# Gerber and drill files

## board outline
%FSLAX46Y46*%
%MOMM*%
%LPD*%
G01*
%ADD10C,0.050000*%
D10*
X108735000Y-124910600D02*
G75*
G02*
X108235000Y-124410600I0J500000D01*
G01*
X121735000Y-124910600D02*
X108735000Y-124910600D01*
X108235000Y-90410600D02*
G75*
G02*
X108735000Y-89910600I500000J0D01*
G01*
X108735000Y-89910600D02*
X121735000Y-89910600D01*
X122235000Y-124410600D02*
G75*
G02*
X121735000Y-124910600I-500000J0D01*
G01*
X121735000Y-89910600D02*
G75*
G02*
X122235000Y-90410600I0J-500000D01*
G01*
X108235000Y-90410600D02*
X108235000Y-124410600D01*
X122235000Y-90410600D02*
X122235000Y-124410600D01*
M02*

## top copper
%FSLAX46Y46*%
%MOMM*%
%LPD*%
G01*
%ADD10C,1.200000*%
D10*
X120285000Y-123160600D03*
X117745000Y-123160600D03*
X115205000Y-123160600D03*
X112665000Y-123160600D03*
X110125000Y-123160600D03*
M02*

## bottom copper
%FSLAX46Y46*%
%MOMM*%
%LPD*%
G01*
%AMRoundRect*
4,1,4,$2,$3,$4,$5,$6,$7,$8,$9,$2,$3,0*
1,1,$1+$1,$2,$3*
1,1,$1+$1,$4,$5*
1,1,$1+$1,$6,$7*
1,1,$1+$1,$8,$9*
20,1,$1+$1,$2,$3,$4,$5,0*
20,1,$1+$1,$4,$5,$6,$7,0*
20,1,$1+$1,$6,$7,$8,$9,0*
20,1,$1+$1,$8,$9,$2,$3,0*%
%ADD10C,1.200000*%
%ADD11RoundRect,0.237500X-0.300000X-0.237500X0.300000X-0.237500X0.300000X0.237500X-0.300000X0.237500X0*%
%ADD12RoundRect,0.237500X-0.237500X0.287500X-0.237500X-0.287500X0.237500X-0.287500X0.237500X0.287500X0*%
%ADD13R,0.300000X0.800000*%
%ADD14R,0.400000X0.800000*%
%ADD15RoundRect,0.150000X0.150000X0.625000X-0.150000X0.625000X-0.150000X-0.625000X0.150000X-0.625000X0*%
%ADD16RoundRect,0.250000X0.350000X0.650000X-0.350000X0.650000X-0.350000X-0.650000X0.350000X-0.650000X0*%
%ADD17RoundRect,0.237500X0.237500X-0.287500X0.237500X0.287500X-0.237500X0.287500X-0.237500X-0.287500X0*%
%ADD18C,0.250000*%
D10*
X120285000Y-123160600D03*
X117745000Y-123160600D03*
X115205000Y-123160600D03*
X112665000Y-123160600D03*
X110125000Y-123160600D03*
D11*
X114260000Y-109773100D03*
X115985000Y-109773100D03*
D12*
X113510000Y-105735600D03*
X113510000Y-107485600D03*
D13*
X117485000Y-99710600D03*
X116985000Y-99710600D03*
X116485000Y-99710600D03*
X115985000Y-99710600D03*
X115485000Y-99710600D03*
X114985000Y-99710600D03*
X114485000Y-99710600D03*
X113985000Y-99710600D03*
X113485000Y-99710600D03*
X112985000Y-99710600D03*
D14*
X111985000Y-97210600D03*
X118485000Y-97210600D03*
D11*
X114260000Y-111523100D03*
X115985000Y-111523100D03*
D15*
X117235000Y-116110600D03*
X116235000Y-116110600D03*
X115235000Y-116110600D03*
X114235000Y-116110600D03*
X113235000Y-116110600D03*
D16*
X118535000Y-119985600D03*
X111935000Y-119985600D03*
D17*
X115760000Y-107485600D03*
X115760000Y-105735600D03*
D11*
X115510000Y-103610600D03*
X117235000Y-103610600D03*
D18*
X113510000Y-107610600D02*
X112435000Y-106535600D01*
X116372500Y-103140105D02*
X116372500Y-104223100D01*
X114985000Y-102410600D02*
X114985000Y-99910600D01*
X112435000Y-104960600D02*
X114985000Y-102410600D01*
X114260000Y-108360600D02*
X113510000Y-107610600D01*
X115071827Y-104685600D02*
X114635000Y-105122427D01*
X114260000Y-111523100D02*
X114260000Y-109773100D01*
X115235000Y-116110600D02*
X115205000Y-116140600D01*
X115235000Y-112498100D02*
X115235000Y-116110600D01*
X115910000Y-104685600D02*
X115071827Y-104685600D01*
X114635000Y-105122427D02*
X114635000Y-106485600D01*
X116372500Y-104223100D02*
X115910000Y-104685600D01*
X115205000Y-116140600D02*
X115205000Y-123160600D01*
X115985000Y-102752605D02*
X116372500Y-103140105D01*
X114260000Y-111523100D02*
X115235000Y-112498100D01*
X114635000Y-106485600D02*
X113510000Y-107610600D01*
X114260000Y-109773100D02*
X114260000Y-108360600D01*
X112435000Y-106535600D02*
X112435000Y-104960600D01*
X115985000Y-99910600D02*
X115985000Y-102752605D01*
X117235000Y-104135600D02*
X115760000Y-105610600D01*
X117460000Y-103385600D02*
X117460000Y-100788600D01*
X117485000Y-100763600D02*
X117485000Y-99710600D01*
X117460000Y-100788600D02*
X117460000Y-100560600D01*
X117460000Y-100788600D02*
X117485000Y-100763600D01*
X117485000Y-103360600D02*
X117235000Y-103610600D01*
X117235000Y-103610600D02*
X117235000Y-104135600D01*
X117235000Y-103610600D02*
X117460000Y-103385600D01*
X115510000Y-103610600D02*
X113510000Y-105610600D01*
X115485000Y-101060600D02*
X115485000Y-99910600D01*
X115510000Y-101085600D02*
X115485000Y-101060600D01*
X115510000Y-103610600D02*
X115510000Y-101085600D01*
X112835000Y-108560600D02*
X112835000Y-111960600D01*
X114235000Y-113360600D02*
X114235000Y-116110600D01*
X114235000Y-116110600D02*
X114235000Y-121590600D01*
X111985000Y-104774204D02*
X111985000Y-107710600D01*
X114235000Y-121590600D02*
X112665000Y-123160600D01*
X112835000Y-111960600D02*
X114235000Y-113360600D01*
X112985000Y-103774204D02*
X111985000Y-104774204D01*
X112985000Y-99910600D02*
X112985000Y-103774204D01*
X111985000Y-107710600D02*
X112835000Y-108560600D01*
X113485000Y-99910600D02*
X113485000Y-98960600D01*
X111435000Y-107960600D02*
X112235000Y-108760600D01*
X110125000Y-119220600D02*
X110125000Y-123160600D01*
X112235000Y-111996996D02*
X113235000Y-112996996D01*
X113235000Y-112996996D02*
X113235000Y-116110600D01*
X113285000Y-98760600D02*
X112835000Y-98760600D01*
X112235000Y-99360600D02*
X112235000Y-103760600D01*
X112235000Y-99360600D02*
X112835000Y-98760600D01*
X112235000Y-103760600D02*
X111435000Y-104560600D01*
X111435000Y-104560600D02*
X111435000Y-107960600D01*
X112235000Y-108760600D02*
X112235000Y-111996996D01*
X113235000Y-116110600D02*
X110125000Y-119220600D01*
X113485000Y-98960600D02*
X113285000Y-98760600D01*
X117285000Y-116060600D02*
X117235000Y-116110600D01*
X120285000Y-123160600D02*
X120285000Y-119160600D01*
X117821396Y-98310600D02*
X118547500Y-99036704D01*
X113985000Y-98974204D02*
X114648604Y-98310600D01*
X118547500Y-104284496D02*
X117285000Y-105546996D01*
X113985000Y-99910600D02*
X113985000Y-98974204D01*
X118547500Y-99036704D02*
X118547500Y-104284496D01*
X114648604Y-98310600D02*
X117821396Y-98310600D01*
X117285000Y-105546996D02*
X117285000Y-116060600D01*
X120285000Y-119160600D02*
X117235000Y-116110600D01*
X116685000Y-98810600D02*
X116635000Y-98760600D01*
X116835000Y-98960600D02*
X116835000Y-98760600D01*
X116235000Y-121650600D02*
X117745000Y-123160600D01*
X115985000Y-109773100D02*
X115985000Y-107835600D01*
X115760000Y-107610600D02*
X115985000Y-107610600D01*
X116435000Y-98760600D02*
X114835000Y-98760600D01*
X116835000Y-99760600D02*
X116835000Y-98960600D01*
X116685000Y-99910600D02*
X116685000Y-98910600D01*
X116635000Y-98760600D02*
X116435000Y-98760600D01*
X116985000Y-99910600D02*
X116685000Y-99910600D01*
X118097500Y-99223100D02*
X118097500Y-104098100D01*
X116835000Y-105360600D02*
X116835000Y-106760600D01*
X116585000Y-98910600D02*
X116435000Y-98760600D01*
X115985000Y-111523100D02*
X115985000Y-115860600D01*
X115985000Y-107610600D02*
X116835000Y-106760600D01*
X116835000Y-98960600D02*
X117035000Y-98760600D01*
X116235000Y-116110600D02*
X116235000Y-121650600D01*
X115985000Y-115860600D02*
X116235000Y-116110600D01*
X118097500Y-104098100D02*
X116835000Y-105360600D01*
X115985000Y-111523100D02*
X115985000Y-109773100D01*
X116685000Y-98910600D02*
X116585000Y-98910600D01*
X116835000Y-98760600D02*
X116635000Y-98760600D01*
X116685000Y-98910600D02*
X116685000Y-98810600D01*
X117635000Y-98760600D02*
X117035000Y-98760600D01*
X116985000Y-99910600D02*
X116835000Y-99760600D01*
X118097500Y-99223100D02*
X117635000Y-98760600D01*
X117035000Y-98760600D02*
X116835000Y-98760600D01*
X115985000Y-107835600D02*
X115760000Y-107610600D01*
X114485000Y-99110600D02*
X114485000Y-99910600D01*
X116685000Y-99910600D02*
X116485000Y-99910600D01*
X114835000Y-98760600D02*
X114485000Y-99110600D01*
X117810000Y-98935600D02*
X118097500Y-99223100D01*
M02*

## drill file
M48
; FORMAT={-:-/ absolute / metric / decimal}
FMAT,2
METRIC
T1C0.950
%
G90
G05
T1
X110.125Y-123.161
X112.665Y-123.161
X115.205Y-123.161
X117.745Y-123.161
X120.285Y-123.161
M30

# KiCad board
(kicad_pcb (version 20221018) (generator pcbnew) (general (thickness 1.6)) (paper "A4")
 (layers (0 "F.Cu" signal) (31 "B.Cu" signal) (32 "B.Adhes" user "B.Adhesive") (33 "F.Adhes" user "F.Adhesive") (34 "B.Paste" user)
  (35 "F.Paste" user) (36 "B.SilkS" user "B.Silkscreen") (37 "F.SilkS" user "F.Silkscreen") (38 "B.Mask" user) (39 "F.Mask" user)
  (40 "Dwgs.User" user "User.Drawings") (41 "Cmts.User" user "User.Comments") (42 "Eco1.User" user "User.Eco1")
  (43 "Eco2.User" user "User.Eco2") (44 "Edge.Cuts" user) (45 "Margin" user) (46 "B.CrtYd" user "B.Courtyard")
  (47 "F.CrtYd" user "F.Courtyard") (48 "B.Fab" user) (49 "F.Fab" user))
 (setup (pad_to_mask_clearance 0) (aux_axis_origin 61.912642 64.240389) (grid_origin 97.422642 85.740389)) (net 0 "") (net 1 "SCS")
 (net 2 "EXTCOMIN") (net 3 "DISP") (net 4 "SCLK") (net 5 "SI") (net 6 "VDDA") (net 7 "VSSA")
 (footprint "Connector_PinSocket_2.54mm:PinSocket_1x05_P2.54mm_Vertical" (layer "F.Cu") (at 120.285 123.1606 -90)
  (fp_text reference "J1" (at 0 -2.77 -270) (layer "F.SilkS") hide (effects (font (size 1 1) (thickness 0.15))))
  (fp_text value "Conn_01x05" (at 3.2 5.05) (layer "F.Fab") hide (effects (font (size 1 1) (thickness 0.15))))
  (pad "1" thru_hole circle (at 0 0 270) (size 1.2 1.2) (drill 0.95) (layers "*.Cu" "*.Mask") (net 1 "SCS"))
  (pad "2" thru_hole circle (at 0 2.54 270) (size 1.2 1.2) (drill 0.95) (layers "*.Cu" "*.Mask") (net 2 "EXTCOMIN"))
  (pad "3" thru_hole circle (at 0 5.08 270) (size 1.2 1.2) (drill 0.95) (layers "*.Cu" "*.Mask") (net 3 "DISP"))
  (pad "4" thru_hole circle (at 0 7.62 270) (size 1.2 1.2) (drill 0.95) (layers "*.Cu" "*.Mask") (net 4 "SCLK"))
  (pad "5" thru_hole circle (at 0 10.16 270) (size 1.2 1.2) (drill 0.95) (layers "*.Cu" "*.Mask") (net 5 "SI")))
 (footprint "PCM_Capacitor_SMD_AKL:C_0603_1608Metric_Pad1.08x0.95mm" (layer "B.Cu") (at 115.1225 109.7731)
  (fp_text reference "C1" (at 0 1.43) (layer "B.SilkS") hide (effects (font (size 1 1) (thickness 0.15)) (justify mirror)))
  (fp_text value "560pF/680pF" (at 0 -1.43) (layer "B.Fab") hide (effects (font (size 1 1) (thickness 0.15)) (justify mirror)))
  (pad "1" smd roundrect (at -0.8625 0) (size 1.075 0.95) (layers "B.Cu" "B.Paste" "B.Mask") (roundrect_rratio 0.25) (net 3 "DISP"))
  (pad "2" smd roundrect (at 0.8625 0) (size 1.075 0.95) (layers "B.Cu" "B.Paste" "B.Mask") (roundrect_rratio 0.25) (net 2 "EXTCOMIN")))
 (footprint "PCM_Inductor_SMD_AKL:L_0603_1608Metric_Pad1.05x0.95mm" (layer "B.Cu") (at 113.51 106.6106 -90)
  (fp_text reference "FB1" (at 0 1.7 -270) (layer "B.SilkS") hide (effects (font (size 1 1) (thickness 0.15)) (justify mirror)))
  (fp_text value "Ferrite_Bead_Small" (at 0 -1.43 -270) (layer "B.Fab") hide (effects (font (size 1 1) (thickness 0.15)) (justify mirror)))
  (pad "1" smd roundrect (at -0.875 0 270) (size 1.05 0.95) (layers "B.Cu" "B.Paste" "B.Mask") (roundrect_rratio 0.25) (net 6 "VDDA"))
  (pad "2" smd roundrect (at 0.875 0 270) (size 1.05 0.95) (layers "B.Cu" "B.Paste" "B.Mask") (roundrect_rratio 0.25) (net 3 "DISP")))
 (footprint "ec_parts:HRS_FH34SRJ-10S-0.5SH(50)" (layer "B.Cu") (at 115.235 98.5606)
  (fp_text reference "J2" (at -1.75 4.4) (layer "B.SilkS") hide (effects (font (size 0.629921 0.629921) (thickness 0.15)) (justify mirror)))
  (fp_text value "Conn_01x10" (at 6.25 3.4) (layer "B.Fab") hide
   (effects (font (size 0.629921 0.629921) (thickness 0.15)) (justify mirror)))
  (pad "1" smd rect (at 2.25 1.15) (size 0.3 0.8) (layers "B.Cu") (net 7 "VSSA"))
  (pad "2" smd rect (at 1.75 1.15) (size 0.3 0.8) (layers "B.Cu") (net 2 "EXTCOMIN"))
  (pad "3" smd rect (at 1.25 1.15) (size 0.3 0.8) (layers "B.Cu") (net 2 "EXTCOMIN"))
  (pad "4" smd rect (at 0.75 1.15) (size 0.3 0.8) (layers "B.Cu") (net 3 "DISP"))
  (pad "5" smd rect (at 0.25 1.15) (size 0.3 0.8) (layers "B.Cu") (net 6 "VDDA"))
  (pad "6" smd rect (at -0.25 1.15) (size 0.3 0.8) (layers "B.Cu") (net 3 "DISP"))
  (pad "7" smd rect (at -0.75 1.15) (size 0.3 0.8) (layers "B.Cu") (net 2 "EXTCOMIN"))
  (pad "8" smd rect (at -1.25 1.15) (size 0.3 0.8) (layers "B.Cu") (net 1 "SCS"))
  (pad "9" smd rect (at -1.75 1.15) (size 0.3 0.8) (layers "B.Cu") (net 5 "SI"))
  (pad "10" smd rect (at -2.25 1.15) (size 0.3 0.8) (layers "B.Cu") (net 4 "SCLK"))
  (pad "MP" smd rect (at -3.25 -1.35) (size 0.4 0.8) (layers "B.Cu" "B.Paste" "B.Mask"))
  (pad "MP" smd rect (at 3.25 -1.35) (size 0.4 0.8) (layers "B.Cu" "B.Paste" "B.Mask")))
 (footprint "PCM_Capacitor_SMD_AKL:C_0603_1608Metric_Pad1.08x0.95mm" (layer "B.Cu") (at 115.1225 111.5231)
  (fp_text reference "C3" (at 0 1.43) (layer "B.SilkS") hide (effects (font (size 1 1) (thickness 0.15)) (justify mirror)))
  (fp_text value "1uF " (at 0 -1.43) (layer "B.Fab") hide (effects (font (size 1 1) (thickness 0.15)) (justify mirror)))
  (pad "1" smd roundrect (at -0.8625 0) (size 1.075 0.95) (layers "B.Cu" "B.Paste" "B.Mask") (roundrect_rratio 0.25) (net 3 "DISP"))
  (pad "2" smd roundrect (at 0.8625 0) (size 1.075 0.95) (layers "B.Cu" "B.Paste" "B.Mask") (roundrect_rratio 0.25) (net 2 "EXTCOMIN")))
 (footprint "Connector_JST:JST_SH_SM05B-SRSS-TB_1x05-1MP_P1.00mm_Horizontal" (layer "B.Cu") (at 115.235 118.1106 180)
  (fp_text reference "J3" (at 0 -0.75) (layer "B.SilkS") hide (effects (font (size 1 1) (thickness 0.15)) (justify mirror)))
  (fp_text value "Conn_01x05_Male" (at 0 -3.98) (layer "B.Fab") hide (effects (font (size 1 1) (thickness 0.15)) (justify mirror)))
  (pad "1" smd roundrect (at -2 2 180) (size 0.6 1.55) (layers "B.Cu" "B.Paste" "B.Mask") (roundrect_rratio 0.25) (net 1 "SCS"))
  (pad "2" smd roundrect (at -1 2 180) (size 0.6 1.55) (layers "B.Cu" "B.Paste" "B.Mask") (roundrect_rratio 0.25) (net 2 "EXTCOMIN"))
  (pad "3" smd roundrect (at 0 2 180) (size 0.6 1.55) (layers "B.Cu" "B.Paste" "B.Mask") (roundrect_rratio 0.25) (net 3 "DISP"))
  (pad "4" smd roundrect (at 1 2 180) (size 0.6 1.55) (layers "B.Cu" "B.Paste" "B.Mask") (roundrect_rratio 0.25) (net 4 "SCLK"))
  (pad "5" smd roundrect (at 2 2 180) (size 0.6 1.55) (layers "B.Cu" "B.Paste" "B.Mask") (roundrect_rratio 0.25) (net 5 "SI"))
  (pad "MP" smd roundrect (at -3.3 -1.875 180) (size 1.2 1.8) (layers "B.Cu" "B.Paste" "B.Mask") (roundrect_rratio 0.2083333333))
  (pad "MP" smd roundrect (at 3.3 -1.875 180) (size 1.2 1.8) (layers "B.Cu" "B.Paste" "B.Mask") (roundrect_rratio 0.2083333333)))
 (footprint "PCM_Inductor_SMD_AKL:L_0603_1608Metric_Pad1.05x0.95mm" (layer "B.Cu") (at 115.76 106.6106 90)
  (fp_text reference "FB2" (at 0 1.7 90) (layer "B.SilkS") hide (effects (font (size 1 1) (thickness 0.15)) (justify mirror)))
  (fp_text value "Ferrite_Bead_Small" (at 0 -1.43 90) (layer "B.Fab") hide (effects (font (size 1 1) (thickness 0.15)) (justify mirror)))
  (pad "1" smd roundrect (at -0.875 0 90) (size 1.05 0.95) (layers "B.Cu" "B.Paste" "B.Mask") (roundrect_rratio 0.25) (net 2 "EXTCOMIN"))
  (pad "2" smd roundrect (at 0.875 0 90) (size 1.05 0.95) (layers "B.Cu" "B.Paste" "B.Mask") (roundrect_rratio 0.25) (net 7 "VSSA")))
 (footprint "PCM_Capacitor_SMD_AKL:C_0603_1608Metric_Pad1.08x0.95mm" (layer "B.Cu") (at 116.3725 103.6106)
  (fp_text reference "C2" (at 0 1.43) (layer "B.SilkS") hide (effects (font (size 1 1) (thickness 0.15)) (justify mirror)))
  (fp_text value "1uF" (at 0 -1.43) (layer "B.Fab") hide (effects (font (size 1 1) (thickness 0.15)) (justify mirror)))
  (pad "1" smd roundrect (at -0.8625 0) (size 1.075 0.95) (layers "B.Cu" "B.Paste" "B.Mask") (roundrect_rratio 0.25) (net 6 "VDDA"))
  (pad "2" smd roundrect (at 0.8625 0) (size 1.075 0.95) (layers "B.Cu" "B.Paste" "B.Mask") (roundrect_rratio 0.25) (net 7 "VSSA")))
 (gr_arc (start 108.735 124.9106) (mid 108.381447 124.764153) (end 108.235 124.4106) (stroke (width 0.05) (type default))
  (layer "Edge.Cuts"))
 (gr_line (start 121.735 124.9106) (end 108.735 124.9106) (stroke (width 0.05) (type solid)) (layer "Edge.Cuts"))
 (gr_arc (start 108.235 90.4106) (mid 108.381447 90.057047) (end 108.735 89.9106) (stroke (width 0.05) (type default)) (layer "Edge.Cuts"))
 (gr_line (start 108.735 89.9106) (end 121.735 89.9106) (stroke (width 0.05) (type solid)) (layer "Edge.Cuts"))
 (gr_arc (start 122.235 124.4106) (mid 122.088553 124.764153) (end 121.735 124.9106) (stroke (width 0.05) (type default))
  (layer "Edge.Cuts"))
 (gr_arc (start 121.735 89.9106) (mid 122.088553 90.057047) (end 122.235 90.4106) (stroke (width 0.05) (type default)) (layer "Edge.Cuts"))
 (gr_line (start 108.235 90.4106) (end 108.235 124.4106) (stroke (width 0.05) (type solid)) (layer "Edge.Cuts"))
 (gr_line (start 122.235 90.4106) (end 122.235 124.4106) (stroke (width 0.05) (type solid)) (layer "Edge.Cuts"))
 (segment (start 113.51 107.6106) (end 112.435 106.5356) (width 0.25) (layer "B.Cu") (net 3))
 (segment (start 116.3725 103.140105) (end 116.3725 104.2231) (width 0.25) (layer "B.Cu") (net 3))
 (segment (start 114.985 102.4106) (end 114.985 99.9106) (width 0.25) (layer "B.Cu") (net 3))
 (segment (start 112.435 104.9606) (end 114.985 102.4106) (width 0.25) (layer "B.Cu") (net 3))
 (segment (start 114.26 108.3606) (end 113.51 107.6106) (width 0.25) (layer "B.Cu") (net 3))
 (segment (start 115.071827 104.6856) (end 114.635 105.122427) (width 0.25) (layer "B.Cu") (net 3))
 (segment (start 114.26 111.5231) (end 114.26 109.7731) (width 0.25) (layer "B.Cu") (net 3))
 (segment (start 115.235 116.1106) (end 115.205 116.1406) (width 0.25) (layer "B.Cu") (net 3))
 (segment (start 115.235 112.4981) (end 115.235 116.1106) (width 0.25) (layer "B.Cu") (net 3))
 (segment (start 115.91 104.6856) (end 115.071827 104.6856) (width 0.25) (layer "B.Cu") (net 3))
 (segment (start 114.635 105.122427) (end 114.635 106.4856) (width 0.25) (layer "B.Cu") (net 3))
 (segment (start 116.3725 104.2231) (end 115.91 104.6856) (width 0.25) (layer "B.Cu") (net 3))
 (segment (start 115.205 116.1406) (end 115.205 123.1606) (width 0.25) (layer "B.Cu") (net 3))
 (segment (start 115.985 102.752605) (end 116.3725 103.140105) (width 0.25) (layer "B.Cu") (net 3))
 (segment (start 114.26 111.5231) (end 115.235 112.4981) (width 0.25) (layer "B.Cu") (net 3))
 (segment (start 114.635 106.4856) (end 113.51 107.6106) (width 0.25) (layer "B.Cu") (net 3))
 (segment (start 114.26 109.7731) (end 114.26 108.3606) (width 0.25) (layer "B.Cu") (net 3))
 (segment (start 112.435 106.5356) (end 112.435 104.9606) (width 0.25) (layer "B.Cu") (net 3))
 (segment (start 115.985 99.9106) (end 115.985 102.752605) (width 0.25) (layer "B.Cu") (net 3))
 (segment (start 117.235 104.1356) (end 115.76 105.6106) (width 0.25) (layer "B.Cu") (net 7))
 (segment (start 117.46 103.3856) (end 117.46 100.7886) (width 0.25) (layer "B.Cu") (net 7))
 (segment (start 117.485 100.7636) (end 117.485 99.7106) (width 0.25) (layer "B.Cu") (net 7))
 (segment (start 117.46 100.7886) (end 117.46 100.5606) (width 0.25) (layer "B.Cu") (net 7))
 (segment (start 117.46 100.7886) (end 117.485 100.7636) (width 0.25) (layer "B.Cu") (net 7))
 (segment (start 117.485 103.3606) (end 117.235 103.6106) (width 0.25) (layer "B.Cu") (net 7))
 (segment (start 117.235 103.6106) (end 117.235 104.1356) (width 0.25) (layer "B.Cu") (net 7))
 (segment (start 117.235 103.6106) (end 117.46 103.3856) (width 0.25) (layer "B.Cu") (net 7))
 (segment (start 115.51 103.6106) (end 113.51 105.6106) (width 0.25) (layer "B.Cu") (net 6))
 (segment (start 115.485 101.0606) (end 115.485 99.9106) (width 0.25) (layer "B.Cu") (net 6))
 (segment (start 115.51 101.0856) (end 115.485 101.0606) (width 0.25) (layer "B.Cu") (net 6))
 (segment (start 115.51 103.6106) (end 115.51 101.0856) (width 0.25) (layer "B.Cu") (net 6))
 (segment (start 112.835 108.5606) (end 112.835 111.9606) (width 0.25) (layer "B.Cu") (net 4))
 (segment (start 114.235 113.3606) (end 114.235 116.1106) (width 0.25) (layer "B.Cu") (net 4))
 (segment (start 114.235 116.1106) (end 114.235 121.5906) (width 0.25) (layer "B.Cu") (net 4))
 (segment (start 111.985 104.774204) (end 111.985 107.7106) (width 0.25) (layer "B.Cu") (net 4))
 (segment (start 114.235 121.5906) (end 112.665 123.1606) (width 0.25) (layer "B.Cu") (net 4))
 (segment (start 112.835 111.9606) (end 114.235 113.3606) (width 0.25) (layer "B.Cu") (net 4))
 (segment (start 112.985 103.774204) (end 111.985 104.774204) (width 0.25) (layer "B.Cu") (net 4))
 (segment (start 112.985 99.9106) (end 112.985 103.774204) (width 0.25) (layer "B.Cu") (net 4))
 (segment (start 111.985 107.7106) (end 112.835 108.5606) (width 0.25) (layer "B.Cu") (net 4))
 (segment (start 113.485 99.9106) (end 113.485 98.9606) (width 0.25) (layer "B.Cu") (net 5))
 (segment (start 111.435 107.9606) (end 112.235 108.7606) (width 0.25) (layer "B.Cu") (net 5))
 (segment (start 110.125 119.2206) (end 110.125 123.1606) (width 0.25) (layer "B.Cu") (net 5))
 (segment (start 112.235 111.996996) (end 113.235 112.996996) (width 0.25) (layer "B.Cu") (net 5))
 (segment (start 113.235 112.996996) (end 113.235 116.1106) (width 0.25) (layer "B.Cu") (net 5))
 (segment (start 113.285 98.7606) (end 112.835 98.7606) (width 0.25) (layer "B.Cu") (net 5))
 (segment (start 112.235 99.3606) (end 112.235 103.7606) (width 0.25) (layer "B.Cu") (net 5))
 (segment (start 112.235 99.3606) (end 112.835 98.7606) (width 0.25) (layer "B.Cu") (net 5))
 (segment (start 112.235 103.7606) (end 111.435 104.5606) (width 0.25) (layer "B.Cu") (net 5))
 (segment (start 111.435 104.5606) (end 111.435 107.9606) (width 0.25) (layer "B.Cu") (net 5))
 (segment (start 112.235 108.7606) (end 112.235 111.996996) (width 0.25) (layer "B.Cu") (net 5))
 (segment (start 113.235 116.1106) (end 110.125 119.2206) (width 0.25) (layer "B.Cu") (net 5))
 (segment (start 113.485 98.9606) (end 113.285 98.7606) (width 0.25) (layer "B.Cu") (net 5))
 (segment (start 117.285 116.0606) (end 117.235 116.1106) (width 0.25) (layer "B.Cu") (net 1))
 (segment (start 120.285 123.1606) (end 120.285 119.1606) (width 0.25) (layer "B.Cu") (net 1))
 (segment (start 117.821396 98.3106) (end 118.5475 99.036704) (width 0.25) (layer "B.Cu") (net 1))
 (segment (start 113.985 98.974204) (end 114.648604 98.3106) (width 0.25) (layer "B.Cu") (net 1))
 (segment (start 118.5475 104.284496) (end 117.285 105.546996) (width 0.25) (layer "B.Cu") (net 1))
 (segment (start 113.985 99.9106) (end 113.985 98.974204) (width 0.25) (layer "B.Cu") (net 1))
 (segment (start 118.5475 99.036704) (end 118.5475 104.284496) (width 0.25) (layer "B.Cu") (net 1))
 (segment (start 114.648604 98.3106) (end 117.821396 98.3106) (width 0.25) (layer "B.Cu") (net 1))
 (segment (start 117.285 105.546996) (end 117.285 116.0606) (width 0.25) (layer "B.Cu") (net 1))
 (segment (start 120.285 119.1606) (end 117.235 116.1106) (width 0.25) (layer "B.Cu") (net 1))
 (segment (start 116.685 98.8106) (end 116.635 98.7606) (width 0.25) (layer "B.Cu") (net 2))
 (segment (start 116.835 98.9606) (end 116.835 98.7606) (width 0.25) (layer "B.Cu") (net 2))
 (segment (start 116.235 121.6506) (end 117.745 123.1606) (width 0.25) (layer "B.Cu") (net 2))
 (segment (start 115.985 109.7731) (end 115.985 107.8356) (width 0.25) (layer "B.Cu") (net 2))
 (segment (start 115.76 107.6106) (end 115.985 107.6106) (width 0.25) (layer "B.Cu") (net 2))
 (segment (start 116.435 98.7606) (end 114.835 98.7606) (width 0.25) (layer "B.Cu") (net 2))
 (segment (start 116.835 99.7606) (end 116.835 98.9606) (width 0.25) (layer "B.Cu") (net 2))
 (segment (start 116.685 99.9106) (end 116.685 98.9106) (width 0.25) (layer "B.Cu") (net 2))
 (segment (start 116.635 98.7606) (end 116.435 98.7606) (width 0.25) (layer "B.Cu") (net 2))
 (segment (start 116.985 99.9106) (end 116.685 99.9106) (width 0.25) (layer "B.Cu") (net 2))
 (segment (start 118.0975 99.2231) (end 118.0975 104.0981) (width 0.25) (layer "B.Cu") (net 2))
 (segment (start 116.835 105.3606) (end 116.835 106.7606) (width 0.25) (layer "B.Cu") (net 2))
 (segment (start 116.585 98.9106) (end 116.435 98.7606) (width 0.25) (layer "B.Cu") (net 2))
 (segment (start 115.985 111.5231) (end 115.985 115.8606) (width 0.25) (layer "B.Cu") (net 2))
 (segment (start 115.985 107.6106) (end 116.835 106.7606) (width 0.25) (layer "B.Cu") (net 2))
 (segment (start 116.835 98.9606) (end 117.035 98.7606) (width 0.25) (layer "B.Cu") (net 2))
 (segment (start 116.235 116.1106) (end 116.235 121.6506) (width 0.25) (layer "B.Cu") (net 2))
 (segment (start 115.985 115.8606) (end 116.235 116.1106) (width 0.25) (layer "B.Cu") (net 2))
 (segment (start 118.0975 104.0981) (end 116.835 105.3606) (width 0.25) (layer "B.Cu") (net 2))
 (segment (start 115.985 111.5231) (end 115.985 109.7731) (width 0.25) (layer "B.Cu") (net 2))
 (segment (start 116.685 98.9106) (end 116.585 98.9106) (width 0.25) (layer "B.Cu") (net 2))
 (segment (start 116.835 98.7606) (end 116.635 98.7606) (width 0.25) (layer "B.Cu") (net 2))
 (segment (start 116.685 98.9106) (end 116.685 98.8106) (width 0.25) (layer "B.Cu") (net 2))
 (segment (start 117.635 98.7606) (end 117.035 98.7606) (width 0.25) (layer "B.Cu") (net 2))
 (segment (start 116.985 99.9106) (end 116.835 99.7606) (width 0.25) (layer "B.Cu") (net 2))
 (segment (start 118.0975 99.2231) (end 117.635 98.7606) (width 0.25) (layer "B.Cu") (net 2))
 (segment (start 117.035 98.7606) (end 116.835 98.7606) (width 0.25) (layer "B.Cu") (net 2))
 (segment (start 115.985 107.8356) (end 115.76 107.6106) (width 0.25) (layer "B.Cu") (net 2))
 (segment (start 114.485 99.1106) (end 114.485 99.9106) (width 0.25) (layer "B.Cu") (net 2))
 (segment (start 116.685 99.9106) (end 116.485 99.9106) (width 0.25) (layer "B.Cu") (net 2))
 (segment (start 114.835 98.7606) (end 114.485 99.1106) (width 0.25) (layer "B.Cu") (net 2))
 (segment (start 117.81 98.9356) (end 118.0975 99.2231) (width 0.25) (layer "B.Cu") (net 2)))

